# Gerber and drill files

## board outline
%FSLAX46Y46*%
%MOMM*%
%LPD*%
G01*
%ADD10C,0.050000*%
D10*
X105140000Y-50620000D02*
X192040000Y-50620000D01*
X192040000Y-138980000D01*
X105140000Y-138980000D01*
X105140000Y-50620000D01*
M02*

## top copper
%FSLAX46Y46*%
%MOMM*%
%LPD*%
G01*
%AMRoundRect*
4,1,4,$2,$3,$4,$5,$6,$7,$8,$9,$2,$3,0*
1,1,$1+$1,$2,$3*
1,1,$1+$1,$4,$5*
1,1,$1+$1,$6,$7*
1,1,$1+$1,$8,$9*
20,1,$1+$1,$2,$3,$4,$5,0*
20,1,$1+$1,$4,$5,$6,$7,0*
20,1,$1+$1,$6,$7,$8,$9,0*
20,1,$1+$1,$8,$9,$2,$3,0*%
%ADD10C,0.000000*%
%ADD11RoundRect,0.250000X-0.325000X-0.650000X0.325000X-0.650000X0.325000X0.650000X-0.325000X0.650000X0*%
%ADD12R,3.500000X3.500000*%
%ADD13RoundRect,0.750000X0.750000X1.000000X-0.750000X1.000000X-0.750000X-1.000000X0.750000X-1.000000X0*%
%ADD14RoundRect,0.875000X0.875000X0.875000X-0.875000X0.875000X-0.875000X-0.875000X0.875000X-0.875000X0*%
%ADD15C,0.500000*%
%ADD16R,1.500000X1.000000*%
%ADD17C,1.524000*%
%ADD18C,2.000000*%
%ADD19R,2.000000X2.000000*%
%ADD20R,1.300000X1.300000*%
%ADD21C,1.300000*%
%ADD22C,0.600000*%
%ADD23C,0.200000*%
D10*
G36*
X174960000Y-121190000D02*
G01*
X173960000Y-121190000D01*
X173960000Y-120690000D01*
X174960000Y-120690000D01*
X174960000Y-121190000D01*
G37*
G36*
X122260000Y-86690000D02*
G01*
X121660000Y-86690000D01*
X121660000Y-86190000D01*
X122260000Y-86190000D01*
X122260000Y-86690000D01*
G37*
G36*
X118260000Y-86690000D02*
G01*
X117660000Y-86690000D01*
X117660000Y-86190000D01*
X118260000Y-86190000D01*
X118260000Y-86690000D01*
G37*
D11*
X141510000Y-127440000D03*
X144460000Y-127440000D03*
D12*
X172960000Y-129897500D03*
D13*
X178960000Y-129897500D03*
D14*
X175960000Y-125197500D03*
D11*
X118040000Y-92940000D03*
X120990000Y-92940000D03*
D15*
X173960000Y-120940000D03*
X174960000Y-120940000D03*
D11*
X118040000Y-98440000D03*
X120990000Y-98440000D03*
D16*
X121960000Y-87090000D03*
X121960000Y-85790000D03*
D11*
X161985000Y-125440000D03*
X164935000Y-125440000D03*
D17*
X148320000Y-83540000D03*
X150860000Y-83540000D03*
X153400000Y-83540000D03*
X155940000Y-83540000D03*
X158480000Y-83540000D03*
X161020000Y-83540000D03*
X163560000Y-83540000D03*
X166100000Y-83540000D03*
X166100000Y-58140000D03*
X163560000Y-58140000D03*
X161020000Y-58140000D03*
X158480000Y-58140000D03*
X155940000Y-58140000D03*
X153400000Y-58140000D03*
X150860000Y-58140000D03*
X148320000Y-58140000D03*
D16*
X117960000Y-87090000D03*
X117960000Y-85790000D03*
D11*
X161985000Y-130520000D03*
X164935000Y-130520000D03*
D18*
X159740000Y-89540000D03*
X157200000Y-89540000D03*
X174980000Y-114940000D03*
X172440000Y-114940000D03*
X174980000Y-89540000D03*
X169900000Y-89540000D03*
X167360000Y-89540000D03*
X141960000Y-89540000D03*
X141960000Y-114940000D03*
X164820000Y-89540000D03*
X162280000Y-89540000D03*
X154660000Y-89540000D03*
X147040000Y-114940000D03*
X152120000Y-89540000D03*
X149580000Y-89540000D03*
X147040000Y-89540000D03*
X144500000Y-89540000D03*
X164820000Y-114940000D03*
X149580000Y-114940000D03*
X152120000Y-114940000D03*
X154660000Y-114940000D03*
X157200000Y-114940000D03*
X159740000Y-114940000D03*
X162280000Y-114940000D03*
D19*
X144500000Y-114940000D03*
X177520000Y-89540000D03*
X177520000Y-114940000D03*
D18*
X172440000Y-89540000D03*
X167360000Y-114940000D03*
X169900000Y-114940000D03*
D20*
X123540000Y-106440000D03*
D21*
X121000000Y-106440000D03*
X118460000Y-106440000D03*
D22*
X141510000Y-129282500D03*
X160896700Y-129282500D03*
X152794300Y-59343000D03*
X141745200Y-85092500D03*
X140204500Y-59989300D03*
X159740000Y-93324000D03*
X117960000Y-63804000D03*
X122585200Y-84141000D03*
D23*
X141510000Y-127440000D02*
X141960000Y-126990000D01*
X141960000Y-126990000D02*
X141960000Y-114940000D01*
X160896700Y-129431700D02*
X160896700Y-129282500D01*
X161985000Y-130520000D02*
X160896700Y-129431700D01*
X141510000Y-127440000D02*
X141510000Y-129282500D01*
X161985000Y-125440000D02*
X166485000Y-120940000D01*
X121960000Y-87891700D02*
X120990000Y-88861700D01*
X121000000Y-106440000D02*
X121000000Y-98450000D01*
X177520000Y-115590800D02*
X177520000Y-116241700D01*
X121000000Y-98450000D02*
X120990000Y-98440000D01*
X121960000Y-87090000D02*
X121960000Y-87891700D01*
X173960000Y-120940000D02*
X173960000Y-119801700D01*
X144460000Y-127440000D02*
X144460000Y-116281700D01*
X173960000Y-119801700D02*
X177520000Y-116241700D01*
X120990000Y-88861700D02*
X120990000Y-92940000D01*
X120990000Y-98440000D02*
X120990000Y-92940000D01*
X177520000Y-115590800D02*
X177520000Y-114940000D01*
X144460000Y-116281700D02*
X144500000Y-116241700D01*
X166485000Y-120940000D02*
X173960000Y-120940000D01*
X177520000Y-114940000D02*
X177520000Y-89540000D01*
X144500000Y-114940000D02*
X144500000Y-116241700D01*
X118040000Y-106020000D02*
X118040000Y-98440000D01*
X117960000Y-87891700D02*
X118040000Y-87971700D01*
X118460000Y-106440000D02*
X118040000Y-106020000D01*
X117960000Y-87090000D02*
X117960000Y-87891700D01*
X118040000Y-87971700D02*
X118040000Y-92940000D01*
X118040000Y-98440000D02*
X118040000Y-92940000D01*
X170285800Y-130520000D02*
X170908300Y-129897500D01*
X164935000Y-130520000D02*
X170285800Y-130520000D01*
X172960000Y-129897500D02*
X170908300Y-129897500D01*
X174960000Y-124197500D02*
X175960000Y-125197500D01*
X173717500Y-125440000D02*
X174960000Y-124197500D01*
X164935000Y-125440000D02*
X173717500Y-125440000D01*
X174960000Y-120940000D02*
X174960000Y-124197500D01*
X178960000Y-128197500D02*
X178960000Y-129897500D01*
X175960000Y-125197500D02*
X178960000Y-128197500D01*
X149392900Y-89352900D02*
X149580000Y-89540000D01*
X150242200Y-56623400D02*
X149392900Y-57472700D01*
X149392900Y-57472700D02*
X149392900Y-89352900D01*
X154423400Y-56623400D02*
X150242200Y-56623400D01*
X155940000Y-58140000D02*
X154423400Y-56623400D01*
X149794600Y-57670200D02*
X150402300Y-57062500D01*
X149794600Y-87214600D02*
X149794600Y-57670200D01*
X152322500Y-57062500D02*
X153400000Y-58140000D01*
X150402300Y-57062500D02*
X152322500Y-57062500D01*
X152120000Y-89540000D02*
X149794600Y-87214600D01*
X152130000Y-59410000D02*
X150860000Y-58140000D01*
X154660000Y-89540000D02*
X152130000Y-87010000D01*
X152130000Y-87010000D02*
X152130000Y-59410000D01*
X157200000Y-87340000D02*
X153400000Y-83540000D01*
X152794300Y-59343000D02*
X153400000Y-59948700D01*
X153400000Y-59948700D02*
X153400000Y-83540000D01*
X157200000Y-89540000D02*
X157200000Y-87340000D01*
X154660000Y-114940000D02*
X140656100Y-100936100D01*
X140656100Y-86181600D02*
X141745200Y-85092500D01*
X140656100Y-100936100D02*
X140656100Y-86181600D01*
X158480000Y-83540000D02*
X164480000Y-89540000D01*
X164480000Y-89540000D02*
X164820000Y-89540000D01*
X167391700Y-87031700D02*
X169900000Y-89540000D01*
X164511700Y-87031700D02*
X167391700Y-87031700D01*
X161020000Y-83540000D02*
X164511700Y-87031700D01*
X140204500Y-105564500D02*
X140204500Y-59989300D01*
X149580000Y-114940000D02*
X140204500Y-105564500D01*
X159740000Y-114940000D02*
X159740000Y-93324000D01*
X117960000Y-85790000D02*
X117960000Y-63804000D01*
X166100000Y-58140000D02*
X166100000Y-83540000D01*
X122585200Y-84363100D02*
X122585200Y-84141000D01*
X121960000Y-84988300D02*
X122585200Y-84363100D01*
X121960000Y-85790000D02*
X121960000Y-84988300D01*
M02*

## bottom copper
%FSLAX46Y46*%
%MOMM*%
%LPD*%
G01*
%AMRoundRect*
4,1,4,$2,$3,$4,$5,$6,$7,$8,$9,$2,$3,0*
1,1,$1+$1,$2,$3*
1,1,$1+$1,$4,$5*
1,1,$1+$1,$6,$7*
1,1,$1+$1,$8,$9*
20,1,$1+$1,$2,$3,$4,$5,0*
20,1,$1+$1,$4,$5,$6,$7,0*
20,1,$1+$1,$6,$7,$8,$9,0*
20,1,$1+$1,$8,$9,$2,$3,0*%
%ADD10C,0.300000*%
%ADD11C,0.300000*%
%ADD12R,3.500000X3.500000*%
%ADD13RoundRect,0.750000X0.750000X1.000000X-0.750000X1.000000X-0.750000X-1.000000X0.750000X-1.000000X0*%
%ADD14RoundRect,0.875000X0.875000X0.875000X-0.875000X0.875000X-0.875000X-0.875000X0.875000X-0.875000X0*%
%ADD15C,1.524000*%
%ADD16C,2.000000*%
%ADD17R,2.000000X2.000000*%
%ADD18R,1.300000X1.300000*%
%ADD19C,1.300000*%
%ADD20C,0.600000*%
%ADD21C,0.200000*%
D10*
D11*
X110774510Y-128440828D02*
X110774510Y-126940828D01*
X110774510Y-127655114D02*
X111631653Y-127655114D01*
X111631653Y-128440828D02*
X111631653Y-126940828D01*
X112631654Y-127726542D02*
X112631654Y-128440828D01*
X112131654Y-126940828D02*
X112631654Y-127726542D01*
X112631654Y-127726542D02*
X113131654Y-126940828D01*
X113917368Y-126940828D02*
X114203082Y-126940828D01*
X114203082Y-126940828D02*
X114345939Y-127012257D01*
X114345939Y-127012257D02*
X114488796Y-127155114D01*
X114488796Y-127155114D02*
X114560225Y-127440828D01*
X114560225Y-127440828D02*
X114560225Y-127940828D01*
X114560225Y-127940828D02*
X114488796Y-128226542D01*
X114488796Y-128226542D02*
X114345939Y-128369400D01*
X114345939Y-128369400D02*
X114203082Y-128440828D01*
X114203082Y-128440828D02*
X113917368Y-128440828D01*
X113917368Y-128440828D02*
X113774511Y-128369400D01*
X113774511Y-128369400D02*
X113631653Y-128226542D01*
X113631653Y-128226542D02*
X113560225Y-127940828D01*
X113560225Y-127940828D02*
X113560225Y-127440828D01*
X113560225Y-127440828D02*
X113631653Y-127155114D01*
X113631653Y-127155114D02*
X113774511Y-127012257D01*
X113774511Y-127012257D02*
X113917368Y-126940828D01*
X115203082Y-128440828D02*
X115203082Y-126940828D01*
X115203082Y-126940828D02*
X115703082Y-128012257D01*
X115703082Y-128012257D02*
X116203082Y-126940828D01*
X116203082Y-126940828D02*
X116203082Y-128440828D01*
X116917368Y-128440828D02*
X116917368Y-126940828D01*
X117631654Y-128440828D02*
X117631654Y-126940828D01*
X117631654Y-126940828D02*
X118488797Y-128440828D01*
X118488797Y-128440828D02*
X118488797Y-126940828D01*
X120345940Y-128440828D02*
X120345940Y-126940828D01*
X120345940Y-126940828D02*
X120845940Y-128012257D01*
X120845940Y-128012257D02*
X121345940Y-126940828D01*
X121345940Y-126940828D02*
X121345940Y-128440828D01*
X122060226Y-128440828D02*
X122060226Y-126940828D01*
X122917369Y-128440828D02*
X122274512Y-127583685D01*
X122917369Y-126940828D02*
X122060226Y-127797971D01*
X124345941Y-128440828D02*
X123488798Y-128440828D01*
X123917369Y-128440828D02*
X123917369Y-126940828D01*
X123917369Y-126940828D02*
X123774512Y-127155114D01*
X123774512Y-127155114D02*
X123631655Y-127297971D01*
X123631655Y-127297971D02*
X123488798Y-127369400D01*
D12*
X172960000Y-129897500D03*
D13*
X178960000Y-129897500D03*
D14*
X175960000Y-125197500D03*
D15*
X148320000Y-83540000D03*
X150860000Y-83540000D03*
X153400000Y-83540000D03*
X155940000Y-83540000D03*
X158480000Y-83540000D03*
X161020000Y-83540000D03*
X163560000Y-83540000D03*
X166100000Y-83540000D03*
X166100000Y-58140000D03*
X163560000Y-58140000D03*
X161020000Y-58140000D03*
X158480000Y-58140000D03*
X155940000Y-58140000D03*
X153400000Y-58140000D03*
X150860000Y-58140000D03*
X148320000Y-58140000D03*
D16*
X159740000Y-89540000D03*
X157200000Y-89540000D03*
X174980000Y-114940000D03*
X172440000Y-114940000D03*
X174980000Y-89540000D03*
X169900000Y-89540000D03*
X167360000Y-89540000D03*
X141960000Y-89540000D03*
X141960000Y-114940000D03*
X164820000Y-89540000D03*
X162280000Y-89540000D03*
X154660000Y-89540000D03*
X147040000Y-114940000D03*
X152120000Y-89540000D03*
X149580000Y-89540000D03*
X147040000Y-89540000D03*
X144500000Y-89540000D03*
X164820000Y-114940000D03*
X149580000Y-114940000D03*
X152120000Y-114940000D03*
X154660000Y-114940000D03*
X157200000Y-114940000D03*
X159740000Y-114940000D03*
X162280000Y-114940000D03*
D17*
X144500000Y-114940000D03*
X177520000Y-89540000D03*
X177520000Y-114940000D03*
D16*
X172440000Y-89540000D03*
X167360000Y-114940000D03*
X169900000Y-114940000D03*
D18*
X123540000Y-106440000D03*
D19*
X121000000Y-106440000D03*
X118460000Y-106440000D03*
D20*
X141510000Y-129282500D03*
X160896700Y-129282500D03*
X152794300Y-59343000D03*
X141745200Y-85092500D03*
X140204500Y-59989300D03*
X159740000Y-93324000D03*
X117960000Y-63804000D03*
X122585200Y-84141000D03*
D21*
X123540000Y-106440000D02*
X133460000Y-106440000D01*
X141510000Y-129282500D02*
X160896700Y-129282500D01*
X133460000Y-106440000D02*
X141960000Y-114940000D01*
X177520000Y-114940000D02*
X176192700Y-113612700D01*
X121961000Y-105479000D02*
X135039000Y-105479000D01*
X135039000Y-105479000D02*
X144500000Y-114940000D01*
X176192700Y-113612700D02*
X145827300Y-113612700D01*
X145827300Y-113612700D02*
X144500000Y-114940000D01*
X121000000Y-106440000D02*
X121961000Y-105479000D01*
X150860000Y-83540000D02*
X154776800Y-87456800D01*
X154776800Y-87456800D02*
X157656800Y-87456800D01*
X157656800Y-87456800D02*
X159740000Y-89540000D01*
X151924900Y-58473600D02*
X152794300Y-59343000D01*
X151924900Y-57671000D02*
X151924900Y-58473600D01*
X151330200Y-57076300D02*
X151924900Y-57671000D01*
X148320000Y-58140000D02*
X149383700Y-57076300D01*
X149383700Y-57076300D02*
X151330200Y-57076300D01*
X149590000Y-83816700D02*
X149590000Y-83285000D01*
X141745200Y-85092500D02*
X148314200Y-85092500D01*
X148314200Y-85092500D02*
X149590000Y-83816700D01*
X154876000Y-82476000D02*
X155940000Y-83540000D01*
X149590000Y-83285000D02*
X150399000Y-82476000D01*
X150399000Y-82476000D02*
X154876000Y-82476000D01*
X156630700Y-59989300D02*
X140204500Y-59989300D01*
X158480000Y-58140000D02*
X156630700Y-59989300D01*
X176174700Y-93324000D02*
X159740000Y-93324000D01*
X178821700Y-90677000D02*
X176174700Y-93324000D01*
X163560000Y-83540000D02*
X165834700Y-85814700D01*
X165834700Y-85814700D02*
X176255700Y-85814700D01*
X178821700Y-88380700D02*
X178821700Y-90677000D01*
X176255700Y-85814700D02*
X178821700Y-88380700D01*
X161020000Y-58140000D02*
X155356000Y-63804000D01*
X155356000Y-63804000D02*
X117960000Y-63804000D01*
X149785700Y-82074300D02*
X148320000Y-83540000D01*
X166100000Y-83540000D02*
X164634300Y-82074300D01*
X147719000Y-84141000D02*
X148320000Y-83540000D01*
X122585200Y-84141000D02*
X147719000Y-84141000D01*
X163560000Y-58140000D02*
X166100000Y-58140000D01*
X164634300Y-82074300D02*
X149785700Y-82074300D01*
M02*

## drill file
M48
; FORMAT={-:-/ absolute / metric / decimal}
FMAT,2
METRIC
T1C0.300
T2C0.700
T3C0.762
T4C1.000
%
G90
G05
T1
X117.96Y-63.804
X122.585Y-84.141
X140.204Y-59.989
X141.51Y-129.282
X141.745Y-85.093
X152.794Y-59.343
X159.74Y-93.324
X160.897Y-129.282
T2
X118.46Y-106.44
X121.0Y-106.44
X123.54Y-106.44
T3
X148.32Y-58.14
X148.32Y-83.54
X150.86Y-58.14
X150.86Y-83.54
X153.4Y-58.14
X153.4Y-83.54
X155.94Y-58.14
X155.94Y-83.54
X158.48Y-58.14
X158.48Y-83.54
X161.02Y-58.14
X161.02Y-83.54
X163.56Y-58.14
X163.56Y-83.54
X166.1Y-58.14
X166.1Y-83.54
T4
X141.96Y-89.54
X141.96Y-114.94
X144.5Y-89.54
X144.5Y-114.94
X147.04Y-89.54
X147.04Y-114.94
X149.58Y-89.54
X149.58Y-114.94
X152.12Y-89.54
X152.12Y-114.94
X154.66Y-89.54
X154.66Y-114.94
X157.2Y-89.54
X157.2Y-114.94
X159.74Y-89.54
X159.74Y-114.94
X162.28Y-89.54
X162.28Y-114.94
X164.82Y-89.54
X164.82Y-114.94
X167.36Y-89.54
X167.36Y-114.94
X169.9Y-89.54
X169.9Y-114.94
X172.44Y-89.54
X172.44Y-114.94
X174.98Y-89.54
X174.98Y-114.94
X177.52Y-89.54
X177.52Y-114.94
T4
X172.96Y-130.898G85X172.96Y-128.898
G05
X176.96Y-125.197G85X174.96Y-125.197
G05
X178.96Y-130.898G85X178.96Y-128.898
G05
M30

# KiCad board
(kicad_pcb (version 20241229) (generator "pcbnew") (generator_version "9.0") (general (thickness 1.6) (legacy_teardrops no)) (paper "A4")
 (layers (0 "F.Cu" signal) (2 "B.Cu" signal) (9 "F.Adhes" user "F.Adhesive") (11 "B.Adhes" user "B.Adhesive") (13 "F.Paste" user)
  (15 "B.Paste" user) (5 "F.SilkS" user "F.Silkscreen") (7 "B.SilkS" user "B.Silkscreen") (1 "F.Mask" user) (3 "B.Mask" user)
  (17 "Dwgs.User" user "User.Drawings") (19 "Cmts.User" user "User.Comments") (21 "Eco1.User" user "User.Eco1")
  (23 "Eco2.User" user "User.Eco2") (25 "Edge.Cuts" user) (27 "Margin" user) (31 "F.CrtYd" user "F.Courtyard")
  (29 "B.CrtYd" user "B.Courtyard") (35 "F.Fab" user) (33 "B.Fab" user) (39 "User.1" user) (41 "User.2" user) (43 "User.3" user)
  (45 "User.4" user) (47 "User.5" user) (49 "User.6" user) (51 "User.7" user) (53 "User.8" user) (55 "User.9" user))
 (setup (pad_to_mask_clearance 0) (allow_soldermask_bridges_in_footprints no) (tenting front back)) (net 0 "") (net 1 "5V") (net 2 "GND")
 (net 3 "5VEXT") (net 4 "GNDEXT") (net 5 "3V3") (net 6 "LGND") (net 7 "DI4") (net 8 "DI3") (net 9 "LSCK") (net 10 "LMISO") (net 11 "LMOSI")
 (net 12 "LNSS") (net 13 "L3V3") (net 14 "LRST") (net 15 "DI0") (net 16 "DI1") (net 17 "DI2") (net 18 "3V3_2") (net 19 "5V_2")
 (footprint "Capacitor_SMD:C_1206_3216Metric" (layer "F.Cu") (at 142.985 127.44)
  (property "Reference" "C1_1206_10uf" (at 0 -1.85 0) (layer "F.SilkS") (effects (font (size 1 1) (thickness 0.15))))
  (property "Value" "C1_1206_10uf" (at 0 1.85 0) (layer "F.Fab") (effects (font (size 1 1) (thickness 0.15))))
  (pad "1" smd roundrect (at -1.475 0) (size 1.15 1.8) (layers "F.Cu" "F.Mask" "F.Paste") (roundrect_rratio 0.217391) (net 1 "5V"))
  (pad "2" smd roundrect (at 1.475 0) (size 1.15 1.8) (layers "F.Cu" "F.Mask" "F.Paste") (roundrect_rratio 0.217391) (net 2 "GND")))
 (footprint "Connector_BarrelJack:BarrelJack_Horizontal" (layer "F.Cu") (at 172.96 129.8975 180)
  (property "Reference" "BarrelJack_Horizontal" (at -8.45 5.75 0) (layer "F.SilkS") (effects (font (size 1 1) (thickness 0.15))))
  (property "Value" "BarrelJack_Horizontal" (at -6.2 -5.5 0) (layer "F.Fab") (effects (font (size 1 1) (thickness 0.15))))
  (pad "1" thru_hole rect (at 0 0 180) (size 3.5 3.5) (drill oval 1 3) (layers "*.Cu" "*.Mask") (remove_unused_layers no) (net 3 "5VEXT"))
  (pad "2" thru_hole roundrect (at -6 0 180) (size 3 3.5) (drill oval 1 3) (layers "*.Cu" "*.Mask") (remove_unused_layers no)
   (roundrect_rratio 0.25) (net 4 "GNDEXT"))
  (pad "3" thru_hole roundrect (at -3 4.7 180) (size 3.5 3.5) (drill oval 3 1) (layers "*.Cu" "*.Mask") (remove_unused_layers no)
   (roundrect_rratio 0.25) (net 4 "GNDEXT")))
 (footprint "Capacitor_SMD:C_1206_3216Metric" (layer "F.Cu") (at 119.515 92.94)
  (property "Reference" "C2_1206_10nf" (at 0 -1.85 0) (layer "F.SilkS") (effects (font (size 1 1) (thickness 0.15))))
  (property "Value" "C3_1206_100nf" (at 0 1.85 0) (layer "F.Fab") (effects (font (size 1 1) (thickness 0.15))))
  (pad "1" smd roundrect (at -1.475 0) (size 1.15 1.8) (layers "F.Cu" "F.Mask" "F.Paste") (roundrect_rratio 0.217391) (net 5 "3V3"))
  (pad "2" smd roundrect (at 1.475 0) (size 1.15 1.8) (layers "F.Cu" "F.Mask" "F.Paste") (roundrect_rratio 0.217391) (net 2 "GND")))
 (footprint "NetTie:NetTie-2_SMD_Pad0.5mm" (layer "F.Cu") (at 174.46 120.94)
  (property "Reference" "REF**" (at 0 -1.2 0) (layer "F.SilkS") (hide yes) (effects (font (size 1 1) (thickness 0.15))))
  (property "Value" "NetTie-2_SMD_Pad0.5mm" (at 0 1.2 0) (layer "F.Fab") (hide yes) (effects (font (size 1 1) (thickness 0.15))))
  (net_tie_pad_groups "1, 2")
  (fp_poly (pts (xy -0.5 -0.25) (xy 0.5 -0.25) (xy 0.5 0.25) (xy -0.5 0.25)) (stroke (width 0) (type solid)) (fill yes) (layer "F.Cu"))
  (pad "1" smd circle (at -0.5 0) (size 0.5 0.5) (layers "F.Cu") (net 2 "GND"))
  (pad "2" smd circle (at 0.5 0) (size 0.5 0.5) (layers "F.Cu") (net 4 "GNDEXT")))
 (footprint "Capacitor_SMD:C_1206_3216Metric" (layer "F.Cu") (at 119.515 98.44)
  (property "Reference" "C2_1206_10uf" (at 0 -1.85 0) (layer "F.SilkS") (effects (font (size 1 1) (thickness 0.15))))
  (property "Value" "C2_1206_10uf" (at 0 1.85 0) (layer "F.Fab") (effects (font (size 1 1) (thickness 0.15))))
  (pad "1" smd roundrect (at -1.475 0) (size 1.15 1.8) (layers "F.Cu" "F.Mask" "F.Paste") (roundrect_rratio 0.217391) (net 5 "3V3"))
  (pad "2" smd roundrect (at 1.475 0) (size 1.15 1.8) (layers "F.Cu" "F.Mask" "F.Paste") (roundrect_rratio 0.217391) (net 2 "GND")))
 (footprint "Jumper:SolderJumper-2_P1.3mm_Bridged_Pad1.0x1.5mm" (layer "F.Cu") (at 121.96 86.44 90)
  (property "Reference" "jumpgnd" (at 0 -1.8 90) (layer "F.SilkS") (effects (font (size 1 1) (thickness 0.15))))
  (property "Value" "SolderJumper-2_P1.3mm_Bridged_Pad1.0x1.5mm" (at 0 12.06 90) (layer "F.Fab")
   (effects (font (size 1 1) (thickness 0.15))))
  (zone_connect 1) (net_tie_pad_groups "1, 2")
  (fp_poly (pts (xy -0.25 -0.3) (xy 0.25 -0.3) (xy 0.25 0.3) (xy -0.25 0.3)) (stroke (width 0) (type solid)) (fill yes) (layer "F.Cu"))
  (pad "1" smd rect (at -0.65 0 90) (size 1 1.5) (layers "F.Cu" "F.Mask") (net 2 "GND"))
  (pad "2" smd rect (at 0.65 0 90) (size 1 1.5) (layers "F.Cu" "F.Mask") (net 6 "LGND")))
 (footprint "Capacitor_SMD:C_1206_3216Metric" (layer "F.Cu") (at 163.46 125.44)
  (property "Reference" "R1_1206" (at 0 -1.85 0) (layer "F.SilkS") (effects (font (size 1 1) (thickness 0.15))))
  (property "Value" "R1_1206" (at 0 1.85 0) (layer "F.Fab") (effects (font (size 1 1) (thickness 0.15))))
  (pad "1" smd roundrect (at -1.475 0) (size 1.15 1.8) (layers "F.Cu" "F.Mask" "F.Paste") (roundrect_rratio 0.217391) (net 2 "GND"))
  (pad "2" smd roundrect (at 1.475 0) (size 1.15 1.8) (layers "F.Cu" "F.Mask" "F.Paste") (roundrect_rratio 0.217391) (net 4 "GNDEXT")))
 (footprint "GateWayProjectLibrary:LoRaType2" (layer "F.Cu") (at 155.94 86.08)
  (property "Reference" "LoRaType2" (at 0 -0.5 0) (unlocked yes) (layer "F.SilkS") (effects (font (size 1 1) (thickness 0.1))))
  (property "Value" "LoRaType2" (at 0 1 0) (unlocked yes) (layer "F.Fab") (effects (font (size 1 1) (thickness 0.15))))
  (pad "1" thru_hole circle (at -7.62 -2.54) (size 1.524 1.524) (drill 0.762) (layers "*.Cu" "*.Mask") (remove_unused_layers no)
   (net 6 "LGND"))
  (pad "2" thru_hole circle (at -5.08 -2.54) (size 1.524 1.524) (drill 0.762) (layers "*.Cu" "*.Mask") (remove_unused_layers no)
   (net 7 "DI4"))
  (pad "3" thru_hole circle (at -2.54 -2.54) (size 1.524 1.524) (drill 0.762) (layers "*.Cu" "*.Mask") (remove_unused_layers no)
   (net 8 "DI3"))
  (pad "4" thru_hole circle (at 0 -2.54) (size 1.524 1.524) (drill 0.762) (layers "*.Cu" "*.Mask") (remove_unused_layers no) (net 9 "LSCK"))
  (pad "5" thru_hole circle (at 2.54 -2.54) (size 1.524 1.524) (drill 0.762) (layers "*.Cu" "*.Mask") (remove_unused_layers no)
   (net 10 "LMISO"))
  (pad "6" thru_hole circle (at 5.08 -2.54) (size 1.524 1.524) (drill 0.762) (layers "*.Cu" "*.Mask") (remove_unused_layers no)
   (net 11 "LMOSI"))
  (pad "7" thru_hole circle (at 7.62 -2.54) (size 1.524 1.524) (drill 0.762) (layers "*.Cu" "*.Mask") (remove_unused_layers no)
   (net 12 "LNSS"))
  (pad "8" thru_hole circle (at 10.16 -2.54) (size 1.524 1.524) (drill 0.762) (layers "*.Cu" "*.Mask") (remove_unused_layers no)
   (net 6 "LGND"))
  (pad "9" thru_hole circle (at 10.16 -27.94) (size 1.524 1.524) (drill 0.762) (layers "*.Cu" "*.Mask") (remove_unused_layers no)
   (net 6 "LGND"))
  (pad "10" thru_hole circle (at 7.62 -27.94) (size 1.524 1.524) (drill 0.762) (layers "*.Cu" "*.Mask") (remove_unused_layers no)
   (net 6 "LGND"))
  (pad "11" thru_hole circle (at 5.08 -27.94) (size 1.524 1.524) (drill 0.762) (layers "*.Cu" "*.Mask") (remove_unused_layers no)
   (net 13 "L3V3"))
  (pad "12" thru_hole circle (at 2.54 -27.94) (size 1.524 1.524) (drill 0.762) (layers "*.Cu" "*.Mask") (remove_unused_layers no)
   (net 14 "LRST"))
  (pad "13" thru_hole circle (at 0 -27.94) (size 1.524 1.524) (drill 0.762) (layers "*.Cu" "*.Mask") (remove_unused_layers no)
   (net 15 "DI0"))
  (pad "14" thru_hole circle (at -2.54 -27.94) (size 1.524 1.524) (drill 0.762) (layers "*.Cu" "*.Mask") (remove_unused_layers no)
   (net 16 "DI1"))
  (pad "15" thru_hole circle (at -5.08 -27.94) (size 1.524 1.524) (drill 0.762) (layers "*.Cu" "*.Mask") (remove_unused_layers no)
   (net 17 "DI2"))
  (pad "16" thru_hole circle (at -7.62 -27.94) (size 1.524 1.524) (drill 0.762) (layers "*.Cu" "*.Mask") (remove_unused_layers no)
   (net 8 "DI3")))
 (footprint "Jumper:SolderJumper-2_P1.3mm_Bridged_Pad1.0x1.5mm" (layer "F.Cu") (at 117.96 86.44 90)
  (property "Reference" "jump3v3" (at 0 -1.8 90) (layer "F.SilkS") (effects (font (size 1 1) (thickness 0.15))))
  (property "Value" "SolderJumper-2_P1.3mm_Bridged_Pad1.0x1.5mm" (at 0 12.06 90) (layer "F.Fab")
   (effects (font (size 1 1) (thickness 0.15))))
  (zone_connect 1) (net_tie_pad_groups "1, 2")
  (fp_poly (pts (xy -0.25 -0.3) (xy 0.25 -0.3) (xy 0.25 0.3) (xy -0.25 0.3)) (stroke (width 0) (type solid)) (fill yes) (layer "F.Cu"))
  (pad "1" smd rect (at -0.65 0 90) (size 1 1.5) (layers "F.Cu" "F.Mask") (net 5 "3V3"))
  (pad "2" smd rect (at 0.65 0 90) (size 1 1.5) (layers "F.Cu" "F.Mask") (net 13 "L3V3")))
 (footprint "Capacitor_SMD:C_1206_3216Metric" (layer "F.Cu") (at 163.46 130.52)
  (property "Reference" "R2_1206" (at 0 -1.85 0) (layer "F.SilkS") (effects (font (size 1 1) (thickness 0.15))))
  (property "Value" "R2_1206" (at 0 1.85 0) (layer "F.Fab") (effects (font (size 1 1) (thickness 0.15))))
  (pad "1" smd roundrect (at -1.475 0) (size 1.15 1.8) (layers "F.Cu" "F.Mask" "F.Paste") (roundrect_rratio 0.217391) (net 1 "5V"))
  (pad "2" smd roundrect (at 1.475 0) (size 1.15 1.8) (layers "F.Cu" "F.Mask" "F.Paste") (roundrect_rratio 0.217391) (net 3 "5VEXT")))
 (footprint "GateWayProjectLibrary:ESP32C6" (layer "F.Cu") (at 159.74 102.24)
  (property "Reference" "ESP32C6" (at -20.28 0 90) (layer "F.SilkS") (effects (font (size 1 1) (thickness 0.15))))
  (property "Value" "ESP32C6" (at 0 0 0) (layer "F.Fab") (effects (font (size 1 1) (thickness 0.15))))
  (pad "0" thru_hole circle (at 0 -12.7) (size 2 2) (drill 1) (layers "*.Cu" "*.Mask") (remove_unused_layers no) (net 7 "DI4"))
  (pad "1" thru_hole circle (at -2.54 -12.7) (size 2 2) (drill 1) (layers "*.Cu" "*.Mask") (remove_unused_layers no) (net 8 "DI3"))
  (pad "2" thru_hole circle (at 15.24 12.7) (size 2 2) (drill 1) (layers "*.Cu" "*.Mask") (remove_unused_layers no))
  (pad "3" thru_hole circle (at 12.7 12.7) (size 2 2) (drill 1) (layers "*.Cu" "*.Mask") (remove_unused_layers no))
  (pad "3V3" thru_hole circle (at 15.24 -12.7) (size 2 2) (drill 1) (layers "*.Cu" "*.Mask") (remove_unused_layers no) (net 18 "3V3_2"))
  (pad "4" thru_hole circle (at 10.16 -12.7) (size 2 2) (drill 1) (layers "*.Cu" "*.Mask") (remove_unused_layers no) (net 11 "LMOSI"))
  (pad "5" thru_hole circle (at 7.62 -12.7) (size 2 2) (drill 1) (layers "*.Cu" "*.Mask") (remove_unused_layers no))
  (pad "5V" thru_hole circle (at -17.78 -12.7) (size 2 2) (drill 1) (layers "*.Cu" "*.Mask") (remove_unused_layers no) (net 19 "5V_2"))
  (pad "5V" thru_hole circle (at -17.78 12.7) (size 2 2) (drill 1) (layers "*.Cu" "*.Mask") (remove_unused_layers no) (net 1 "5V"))
  (pad "6" thru_hole circle (at 5.08 -12.7) (size 2 2) (drill 1) (layers "*.Cu" "*.Mask") (remove_unused_layers no) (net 10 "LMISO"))
  (pad "7" thru_hole circle (at 2.54 -12.7) (size 2 2) (drill 1) (layers "*.Cu" "*.Mask") (remove_unused_layers no))
  (pad "8" thru_hole circle (at -5.08 -12.7) (size 2 2) (drill 1) (layers "*.Cu" "*.Mask") (remove_unused_layers no) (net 17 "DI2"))
  (pad "9" thru_hole circle (at -12.7 12.7) (size 2 2) (drill 1) (layers "*.Cu" "*.Mask") (remove_unused_layers no))
  (pad "10" thru_hole circle (at -7.62 -12.7) (size 2 2) (drill 1) (layers "*.Cu" "*.Mask") (remove_unused_layers no) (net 16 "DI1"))
  (pad "11" thru_hole circle (at -10.16 -12.7) (size 2 2) (drill 1) (layers "*.Cu" "*.Mask") (remove_unused_layers no) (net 15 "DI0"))
  (pad "12" thru_hole circle (at -12.7 -12.7) (size 2 2) (drill 1) (layers "*.Cu" "*.Mask") (remove_unused_layers no))
  (pad "13" thru_hole circle (at -15.24 -12.7) (size 2 2) (drill 1) (layers "*.Cu" "*.Mask") (remove_unused_layers no))
  (pad "15" thru_hole circle (at 5.08 12.7) (size 2 2) (drill 1) (layers "*.Cu" "*.Mask") (remove_unused_layers no))
  (pad "18" thru_hole circle (at -10.16 12.7) (size 2 2) (drill 1) (layers "*.Cu" "*.Mask") (remove_unused_layers no) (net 14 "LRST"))
  (pad "19" thru_hole circle (at -7.62 12.7) (size 2 2) (drill 1) (layers "*.Cu" "*.Mask") (remove_unused_layers no))
  (pad "20" thru_hole circle (at -5.08 12.7) (size 2 2) (drill 1) (layers "*.Cu" "*.Mask") (remove_unused_layers no) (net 9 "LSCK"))
  (pad "21" thru_hole circle (at -2.54 12.7) (size 2 2) (drill 1) (layers "*.Cu" "*.Mask") (remove_unused_layers no))
  (pad "22" thru_hole circle (at 0 12.7) (size 2 2) (drill 1) (layers "*.Cu" "*.Mask") (remove_unused_layers no) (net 12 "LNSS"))
  (pad "23" thru_hole circle (at 2.54 12.7) (size 2 2) (drill 1) (layers "*.Cu" "*.Mask") (remove_unused_layers no))
  (pad "GND" thru_hole rect (at -15.24 12.7) (size 2 2) (drill 1) (layers "*.Cu" "*.Mask") (remove_unused_layers no) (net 2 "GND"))
  (pad "GND" thru_hole rect (at 17.78 -12.7) (size 2 2) (drill 1) (layers "*.Cu" "*.Mask") (remove_unused_layers no) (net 2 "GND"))
  (pad "GND" thru_hole rect (at 17.78 12.7) (size 2 2) (drill 1) (layers "*.Cu" "*.Mask") (remove_unused_layers no) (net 2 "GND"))
  (pad "RST" thru_hole circle (at 12.7 -12.7) (size 2 2) (drill 1) (layers "*.Cu" "*.Mask") (remove_unused_layers no))
  (pad "RX" thru_hole circle (at 7.62 12.7) (size 2 2) (drill 1) (layers "*.Cu" "*.Mask") (remove_unused_layers no))
  (pad "TX" thru_hole circle (at 10.16 12.7) (size 2 2) (drill 1) (layers "*.Cu" "*.Mask") (remove_unused_layers no)))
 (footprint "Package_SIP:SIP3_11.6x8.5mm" (layer "F.Cu") (at 123.54 106.44 180)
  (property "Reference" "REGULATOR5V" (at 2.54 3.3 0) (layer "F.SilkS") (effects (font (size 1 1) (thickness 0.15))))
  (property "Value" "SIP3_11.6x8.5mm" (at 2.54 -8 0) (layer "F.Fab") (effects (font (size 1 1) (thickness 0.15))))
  (pad "1" thru_hole rect (at 0 0 90) (size 1.3 1.3) (drill 0.7) (layers "*.Cu" "*.Mask") (remove_unused_layers no) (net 1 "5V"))
  (pad "2" thru_hole circle (at 2.54 0) (size 1.3 1.3) (drill 0.7) (layers "*.Cu" "*.Mask") (remove_unused_layers no) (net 2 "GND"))
  (pad "3" thru_hole circle (at 5.08 0 90) (size 1.3 1.3) (drill 0.7) (layers "*.Cu" "*.Mask") (remove_unused_layers no) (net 5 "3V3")))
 (gr_rect (start 105.14 50.62) (end 192.04 138.98) (stroke (width 0.05) (type default)) (fill no) (layer "Edge.Cuts"))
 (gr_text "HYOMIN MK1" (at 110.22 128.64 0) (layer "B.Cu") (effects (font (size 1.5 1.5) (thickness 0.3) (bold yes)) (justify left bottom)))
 (segment (start 141.51 127.44) (end 141.96 126.99) (width 0.2) (layer "F.Cu") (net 1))
 (segment (start 141.96 126.99) (end 141.96 114.94) (width 0.2) (layer "F.Cu") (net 1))
 (segment (start 160.8967 129.4317) (end 160.8967 129.2825) (width 0.2) (layer "F.Cu") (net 1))
 (segment (start 161.985 130.52) (end 160.8967 129.4317) (width 0.2) (layer "F.Cu") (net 1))
 (segment (start 141.51 127.44) (end 141.51 129.2825) (width 0.2) (layer "F.Cu") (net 1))
 (via (at 141.51 129.2825) (size 0.6) (drill 0.3) (layers "F.Cu" "B.Cu") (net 1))
 (via (at 160.8967 129.2825) (size 0.6) (drill 0.3) (layers "F.Cu" "B.Cu") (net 1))
 (segment (start 123.54 106.44) (end 133.46 106.44) (width 0.2) (layer "B.Cu") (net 1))
 (segment (start 141.51 129.2825) (end 160.8967 129.2825) (width 0.2) (layer "B.Cu") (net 1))
 (segment (start 133.46 106.44) (end 141.96 114.94) (width 0.2) (layer "B.Cu") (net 1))
 (segment (start 161.985 125.44) (end 166.485 120.94) (width 0.2) (layer "F.Cu") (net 2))
 (segment (start 121.96 87.8917) (end 120.99 88.8617) (width 0.2) (layer "F.Cu") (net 2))
 (segment (start 121 106.44) (end 121 98.45) (width 0.2) (layer "F.Cu") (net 2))
 (segment (start 177.52 115.5908) (end 177.52 116.2417) (width 0.2) (layer "F.Cu") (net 2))
 (segment (start 121 98.45) (end 120.99 98.44) (width 0.2) (layer "F.Cu") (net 2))
 (segment (start 121.96 87.09) (end 121.96 87.8917) (width 0.2) (layer "F.Cu") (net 2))
 (segment (start 173.96 120.94) (end 173.96 119.8017) (width 0.2) (layer "F.Cu") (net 2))
 (segment (start 144.46 127.44) (end 144.46 116.2817) (width 0.2) (layer "F.Cu") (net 2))
 (segment (start 173.96 119.8017) (end 177.52 116.2417) (width 0.2) (layer "F.Cu") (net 2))
 (segment (start 120.99 88.8617) (end 120.99 92.94) (width 0.2) (layer "F.Cu") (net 2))
 (segment (start 120.99 98.44) (end 120.99 92.94) (width 0.2) (layer "F.Cu") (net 2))
 (segment (start 177.52 115.5908) (end 177.52 114.94) (width 0.2) (layer "F.Cu") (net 2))
 (segment (start 144.46 116.2817) (end 144.5 116.2417) (width 0.2) (layer "F.Cu") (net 2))
 (segment (start 166.485 120.94) (end 173.96 120.94) (width 0.2) (layer "F.Cu") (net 2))
 (segment (start 177.52 114.94) (end 177.52 89.54) (width 0.2) (layer "F.Cu") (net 2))
 (segment (start 144.5 114.94) (end 144.5 116.2417) (width 0.2) (layer "F.Cu") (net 2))
 (segment (start 177.52 114.94) (end 176.1927 113.6127) (width 0.2) (layer "B.Cu") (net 2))
 (segment (start 121.961 105.479) (end 135.039 105.479) (width 0.2) (layer "B.Cu") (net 2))
 (segment (start 135.039 105.479) (end 144.5 114.94) (width 0.2) (layer "B.Cu") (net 2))
 (segment (start 176.1927 113.6127) (end 145.8273 113.6127) (width 0.2) (layer "B.Cu") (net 2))
 (segment (start 145.8273 113.6127) (end 144.5 114.94) (width 0.2) (layer "B.Cu") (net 2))
 (segment (start 121 106.44) (end 121.961 105.479) (width 0.2) (layer "B.Cu") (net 2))
 (segment (start 118.04 106.02) (end 118.04 98.44) (width 0.2) (layer "F.Cu") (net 5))
 (segment (start 117.96 87.8917) (end 118.04 87.9717) (width 0.2) (layer "F.Cu") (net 5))
 (segment (start 118.46 106.44) (end 118.04 106.02) (width 0.2) (layer "F.Cu") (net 5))
 (segment (start 117.96 87.09) (end 117.96 87.8917) (width 0.2) (layer "F.Cu") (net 5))
 (segment (start 118.04 87.9717) (end 118.04 92.94) (width 0.2) (layer "F.Cu") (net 5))
 (segment (start 118.04 98.44) (end 118.04 92.94) (width 0.2) (layer "F.Cu") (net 5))
 (segment (start 170.2858 130.52) (end 170.9083 129.8975) (width 0.2) (layer "F.Cu") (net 3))
 (segment (start 164.935 130.52) (end 170.2858 130.52) (width 0.2) (layer "F.Cu") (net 3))
 (segment (start 172.96 129.8975) (end 170.9083 129.8975) (width 0.2) (layer "F.Cu") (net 3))
 (segment (start 174.96 124.1975) (end 175.96 125.1975) (width 0.2) (layer "F.Cu") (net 4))
 (segment (start 173.7175 125.44) (end 174.96 124.1975) (width 0.2) (layer "F.Cu") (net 4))
 (segment (start 164.935 125.44) (end 173.7175 125.44) (width 0.2) (layer "F.Cu") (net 4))
 (segment (start 174.96 120.94) (end 174.96 124.1975) (width 0.2) (layer "F.Cu") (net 4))
 (segment (start 178.96 128.1975) (end 178.96 129.8975) (width 0.2) (layer "F.Cu") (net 4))
 (segment (start 175.96 125.1975) (end 178.96 128.1975) (width 0.2) (layer "F.Cu") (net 4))
 (segment (start 150.86 83.54) (end 154.7768 87.4568) (width 0.2) (layer "B.Cu") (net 7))
 (segment (start 154.7768 87.4568) (end 157.6568 87.4568) (width 0.2) (layer "B.Cu") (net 7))
 (segment (start 157.6568 87.4568) (end 159.74 89.54) (width 0.2) (layer "B.Cu") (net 7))
 (segment (start 149.3929 89.3529) (end 149.58 89.54) (width 0.2) (layer "F.Cu") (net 15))
 (segment (start 150.2422 56.6234) (end 149.3929 57.4727) (width 0.2) (layer "F.Cu") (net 15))
 (segment (start 149.3929 57.4727) (end 149.3929 89.3529) (width 0.2) (layer "F.Cu") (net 15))
 (segment (start 154.4234 56.6234) (end 150.2422 56.6234) (width 0.2) (layer "F.Cu") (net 15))
 (segment (start 155.94 58.14) (end 154.4234 56.6234) (width 0.2) (layer "F.Cu") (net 15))
 (segment (start 149.7946 57.6702) (end 150.4023 57.0625) (width 0.2) (layer "F.Cu") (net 16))
 (segment (start 149.7946 87.2146) (end 149.7946 57.6702) (width 0.2) (layer "F.Cu") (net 16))
 (segment (start 152.3225 57.0625) (end 153.4 58.14) (width 0.2) (layer "F.Cu") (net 16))
 (segment (start 150.4023 57.0625) (end 152.3225 57.0625) (width 0.2) (layer "F.Cu") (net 16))
 (segment (start 152.12 89.54) (end 149.7946 87.2146) (width 0.2) (layer "F.Cu") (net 16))
 (segment (start 152.13 59.41) (end 150.86 58.14) (width 0.2) (layer "F.Cu") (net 17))
 (segment (start 154.66 89.54) (end 152.13 87.01) (width 0.2) (layer "F.Cu") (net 17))
 (segment (start 152.13 87.01) (end 152.13 59.41) (width 0.2) (layer "F.Cu") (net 17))
 (segment (start 157.2 87.34) (end 153.4 83.54) (width 0.2) (layer "F.Cu") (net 8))
 (segment (start 152.7943 59.343) (end 153.4 59.9487) (width 0.2) (layer "F.Cu") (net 8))
 (segment (start 153.4 59.9487) (end 153.4 83.54) (width 0.2) (layer "F.Cu") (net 8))
 (segment (start 157.2 89.54) (end 157.2 87.34) (width 0.2) (layer "F.Cu") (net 8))
 (via (at 152.7943 59.343) (size 0.6) (drill 0.3) (layers "F.Cu" "B.Cu") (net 8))
 (segment (start 151.9249 58.4736) (end 152.7943 59.343) (width 0.2) (layer "B.Cu") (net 8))
 (segment (start 151.9249 57.671) (end 151.9249 58.4736) (width 0.2) (layer "B.Cu") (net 8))
 (segment (start 151.3302 57.0763) (end 151.9249 57.671) (width 0.2) (layer "B.Cu") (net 8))
 (segment (start 148.32 58.14) (end 149.3837 57.0763) (width 0.2) (layer "B.Cu") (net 8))
 (segment (start 149.3837 57.0763) (end 151.3302 57.0763) (width 0.2) (layer "B.Cu") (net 8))
 (segment (start 154.66 114.94) (end 140.6561 100.9361) (width 0.2) (layer "F.Cu") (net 9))
 (segment (start 140.6561 86.1816) (end 141.7452 85.0925) (width 0.2) (layer "F.Cu") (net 9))
 (segment (start 140.6561 100.9361) (end 140.6561 86.1816) (width 0.2) (layer "F.Cu") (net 9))
 (via (at 141.7452 85.0925) (size 0.6) (drill 0.3) (layers "F.Cu" "B.Cu") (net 9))
 (segment (start 149.59 83.8167) (end 149.59 83.285) (width 0.2) (layer "B.Cu") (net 9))
 (segment (start 141.7452 85.0925) (end 148.3142 85.0925) (width 0.2) (layer "B.Cu") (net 9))
 (segment (start 148.3142 85.0925) (end 149.59 83.8167) (width 0.2) (layer "B.Cu") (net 9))
 (segment (start 154.876 82.476) (end 155.94 83.54) (width 0.2) (layer "B.Cu") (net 9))
 (segment (start 149.59 83.285) (end 150.399 82.476) (width 0.2) (layer "B.Cu") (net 9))
 (segment (start 150.399 82.476) (end 154.876 82.476) (width 0.2) (layer "B.Cu") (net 9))
 (segment (start 158.48 83.54) (end 164.48 89.54) (width 0.2) (layer "F.Cu") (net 10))
 (segment (start 164.48 89.54) (end 164.82 89.54) (width 0.2) (layer "F.Cu") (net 10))
 (segment (start 167.3917 87.0317) (end 169.9 89.54) (width 0.2) (layer "F.Cu") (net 11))
 (segment (start 164.5117 87.0317) (end 167.3917 87.0317) (width 0.2) (layer "F.Cu") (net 11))
 (segment (start 161.02 83.54) (end 164.5117 87.0317) (width 0.2) (layer "F.Cu") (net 11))
 (segment (start 140.2045 105.5645) (end 140.2045 59.9893) (width 0.2) (layer "F.Cu") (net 14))
 (segment (start 149.58 114.94) (end 140.2045 105.5645) (width 0.2) (layer "F.Cu") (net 14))
 (via (at 140.2045 59.9893) (size 0.6) (drill 0.3) (layers "F.Cu" "B.Cu") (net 14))
 (segment (start 156.6307 59.9893) (end 140.2045 59.9893) (width 0.2) (layer "B.Cu") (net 14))
 (segment (start 158.48 58.14) (end 156.6307 59.9893) (width 0.2) (layer "B.Cu") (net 14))
 (segment (start 159.74 114.94) (end 159.74 93.324) (width 0.2) (layer "F.Cu") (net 12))
 (via (at 159.74 93.324) (size 0.6) (drill 0.3) (layers "F.Cu" "B.Cu") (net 12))
 (segment (start 176.1747 93.324) (end 159.74 93.324) (width 0.2) (layer "B.Cu") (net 12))
 (segment (start 178.8217 90.677) (end 176.1747 93.324) (width 0.2) (layer "B.Cu") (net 12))
 (segment (start 163.56 83.54) (end 165.8347 85.8147) (width 0.2) (layer "B.Cu") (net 12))
 (segment (start 165.8347 85.8147) (end 176.2557 85.8147) (width 0.2) (layer "B.Cu") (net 12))
 (segment (start 178.8217 88.3807) (end 178.8217 90.677) (width 0.2) (layer "B.Cu") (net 12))
 (segment (start 176.2557 85.8147) (end 178.8217 88.3807) (width 0.2) (layer "B.Cu") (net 12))
 (segment (start 117.96 85.79) (end 117.96 63.804) (width 0.2) (layer "F.Cu") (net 13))
 (via (at 117.96 63.804) (size 0.6) (drill 0.3) (layers "F.Cu" "B.Cu") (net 13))
 (segment (start 161.02 58.14) (end 155.356 63.804) (width 0.2) (layer "B.Cu") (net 13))
 (segment (start 155.356 63.804) (end 117.96 63.804) (width 0.2) (layer "B.Cu") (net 13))
 (segment (start 166.1 58.14) (end 166.1 83.54) (width 0.2) (layer "F.Cu") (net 6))
 (segment (start 122.5852 84.3631) (end 122.5852 84.141) (width 0.2) (layer "F.Cu") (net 6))
 (segment (start 121.96 84.9883) (end 122.5852 84.3631) (width 0.2) (layer "F.Cu") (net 6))
 (segment (start 121.96 85.79) (end 121.96 84.9883) (width 0.2) (layer "F.Cu") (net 6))
 (via (at 122.5852 84.141) (size 0.6) (drill 0.3) (layers "F.Cu" "B.Cu") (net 6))
 (segment (start 149.7857 82.0743) (end 148.32 83.54) (width 0.2) (layer "B.Cu") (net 6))
 (segment (start 166.1 83.54) (end 164.6343 82.0743) (width 0.2) (layer "B.Cu") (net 6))
 (segment (start 147.719 84.141) (end 148.32 83.54) (width 0.2) (layer "B.Cu") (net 6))
 (segment (start 122.5852 84.141) (end 147.719 84.141) (width 0.2) (layer "B.Cu") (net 6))
 (segment (start 163.56 58.14) (end 166.1 58.14) (width 0.2) (layer "B.Cu") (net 6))
 (segment (start 164.6343 82.0743) (end 149.7857 82.0743) (width 0.2) (layer "B.Cu") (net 6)))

